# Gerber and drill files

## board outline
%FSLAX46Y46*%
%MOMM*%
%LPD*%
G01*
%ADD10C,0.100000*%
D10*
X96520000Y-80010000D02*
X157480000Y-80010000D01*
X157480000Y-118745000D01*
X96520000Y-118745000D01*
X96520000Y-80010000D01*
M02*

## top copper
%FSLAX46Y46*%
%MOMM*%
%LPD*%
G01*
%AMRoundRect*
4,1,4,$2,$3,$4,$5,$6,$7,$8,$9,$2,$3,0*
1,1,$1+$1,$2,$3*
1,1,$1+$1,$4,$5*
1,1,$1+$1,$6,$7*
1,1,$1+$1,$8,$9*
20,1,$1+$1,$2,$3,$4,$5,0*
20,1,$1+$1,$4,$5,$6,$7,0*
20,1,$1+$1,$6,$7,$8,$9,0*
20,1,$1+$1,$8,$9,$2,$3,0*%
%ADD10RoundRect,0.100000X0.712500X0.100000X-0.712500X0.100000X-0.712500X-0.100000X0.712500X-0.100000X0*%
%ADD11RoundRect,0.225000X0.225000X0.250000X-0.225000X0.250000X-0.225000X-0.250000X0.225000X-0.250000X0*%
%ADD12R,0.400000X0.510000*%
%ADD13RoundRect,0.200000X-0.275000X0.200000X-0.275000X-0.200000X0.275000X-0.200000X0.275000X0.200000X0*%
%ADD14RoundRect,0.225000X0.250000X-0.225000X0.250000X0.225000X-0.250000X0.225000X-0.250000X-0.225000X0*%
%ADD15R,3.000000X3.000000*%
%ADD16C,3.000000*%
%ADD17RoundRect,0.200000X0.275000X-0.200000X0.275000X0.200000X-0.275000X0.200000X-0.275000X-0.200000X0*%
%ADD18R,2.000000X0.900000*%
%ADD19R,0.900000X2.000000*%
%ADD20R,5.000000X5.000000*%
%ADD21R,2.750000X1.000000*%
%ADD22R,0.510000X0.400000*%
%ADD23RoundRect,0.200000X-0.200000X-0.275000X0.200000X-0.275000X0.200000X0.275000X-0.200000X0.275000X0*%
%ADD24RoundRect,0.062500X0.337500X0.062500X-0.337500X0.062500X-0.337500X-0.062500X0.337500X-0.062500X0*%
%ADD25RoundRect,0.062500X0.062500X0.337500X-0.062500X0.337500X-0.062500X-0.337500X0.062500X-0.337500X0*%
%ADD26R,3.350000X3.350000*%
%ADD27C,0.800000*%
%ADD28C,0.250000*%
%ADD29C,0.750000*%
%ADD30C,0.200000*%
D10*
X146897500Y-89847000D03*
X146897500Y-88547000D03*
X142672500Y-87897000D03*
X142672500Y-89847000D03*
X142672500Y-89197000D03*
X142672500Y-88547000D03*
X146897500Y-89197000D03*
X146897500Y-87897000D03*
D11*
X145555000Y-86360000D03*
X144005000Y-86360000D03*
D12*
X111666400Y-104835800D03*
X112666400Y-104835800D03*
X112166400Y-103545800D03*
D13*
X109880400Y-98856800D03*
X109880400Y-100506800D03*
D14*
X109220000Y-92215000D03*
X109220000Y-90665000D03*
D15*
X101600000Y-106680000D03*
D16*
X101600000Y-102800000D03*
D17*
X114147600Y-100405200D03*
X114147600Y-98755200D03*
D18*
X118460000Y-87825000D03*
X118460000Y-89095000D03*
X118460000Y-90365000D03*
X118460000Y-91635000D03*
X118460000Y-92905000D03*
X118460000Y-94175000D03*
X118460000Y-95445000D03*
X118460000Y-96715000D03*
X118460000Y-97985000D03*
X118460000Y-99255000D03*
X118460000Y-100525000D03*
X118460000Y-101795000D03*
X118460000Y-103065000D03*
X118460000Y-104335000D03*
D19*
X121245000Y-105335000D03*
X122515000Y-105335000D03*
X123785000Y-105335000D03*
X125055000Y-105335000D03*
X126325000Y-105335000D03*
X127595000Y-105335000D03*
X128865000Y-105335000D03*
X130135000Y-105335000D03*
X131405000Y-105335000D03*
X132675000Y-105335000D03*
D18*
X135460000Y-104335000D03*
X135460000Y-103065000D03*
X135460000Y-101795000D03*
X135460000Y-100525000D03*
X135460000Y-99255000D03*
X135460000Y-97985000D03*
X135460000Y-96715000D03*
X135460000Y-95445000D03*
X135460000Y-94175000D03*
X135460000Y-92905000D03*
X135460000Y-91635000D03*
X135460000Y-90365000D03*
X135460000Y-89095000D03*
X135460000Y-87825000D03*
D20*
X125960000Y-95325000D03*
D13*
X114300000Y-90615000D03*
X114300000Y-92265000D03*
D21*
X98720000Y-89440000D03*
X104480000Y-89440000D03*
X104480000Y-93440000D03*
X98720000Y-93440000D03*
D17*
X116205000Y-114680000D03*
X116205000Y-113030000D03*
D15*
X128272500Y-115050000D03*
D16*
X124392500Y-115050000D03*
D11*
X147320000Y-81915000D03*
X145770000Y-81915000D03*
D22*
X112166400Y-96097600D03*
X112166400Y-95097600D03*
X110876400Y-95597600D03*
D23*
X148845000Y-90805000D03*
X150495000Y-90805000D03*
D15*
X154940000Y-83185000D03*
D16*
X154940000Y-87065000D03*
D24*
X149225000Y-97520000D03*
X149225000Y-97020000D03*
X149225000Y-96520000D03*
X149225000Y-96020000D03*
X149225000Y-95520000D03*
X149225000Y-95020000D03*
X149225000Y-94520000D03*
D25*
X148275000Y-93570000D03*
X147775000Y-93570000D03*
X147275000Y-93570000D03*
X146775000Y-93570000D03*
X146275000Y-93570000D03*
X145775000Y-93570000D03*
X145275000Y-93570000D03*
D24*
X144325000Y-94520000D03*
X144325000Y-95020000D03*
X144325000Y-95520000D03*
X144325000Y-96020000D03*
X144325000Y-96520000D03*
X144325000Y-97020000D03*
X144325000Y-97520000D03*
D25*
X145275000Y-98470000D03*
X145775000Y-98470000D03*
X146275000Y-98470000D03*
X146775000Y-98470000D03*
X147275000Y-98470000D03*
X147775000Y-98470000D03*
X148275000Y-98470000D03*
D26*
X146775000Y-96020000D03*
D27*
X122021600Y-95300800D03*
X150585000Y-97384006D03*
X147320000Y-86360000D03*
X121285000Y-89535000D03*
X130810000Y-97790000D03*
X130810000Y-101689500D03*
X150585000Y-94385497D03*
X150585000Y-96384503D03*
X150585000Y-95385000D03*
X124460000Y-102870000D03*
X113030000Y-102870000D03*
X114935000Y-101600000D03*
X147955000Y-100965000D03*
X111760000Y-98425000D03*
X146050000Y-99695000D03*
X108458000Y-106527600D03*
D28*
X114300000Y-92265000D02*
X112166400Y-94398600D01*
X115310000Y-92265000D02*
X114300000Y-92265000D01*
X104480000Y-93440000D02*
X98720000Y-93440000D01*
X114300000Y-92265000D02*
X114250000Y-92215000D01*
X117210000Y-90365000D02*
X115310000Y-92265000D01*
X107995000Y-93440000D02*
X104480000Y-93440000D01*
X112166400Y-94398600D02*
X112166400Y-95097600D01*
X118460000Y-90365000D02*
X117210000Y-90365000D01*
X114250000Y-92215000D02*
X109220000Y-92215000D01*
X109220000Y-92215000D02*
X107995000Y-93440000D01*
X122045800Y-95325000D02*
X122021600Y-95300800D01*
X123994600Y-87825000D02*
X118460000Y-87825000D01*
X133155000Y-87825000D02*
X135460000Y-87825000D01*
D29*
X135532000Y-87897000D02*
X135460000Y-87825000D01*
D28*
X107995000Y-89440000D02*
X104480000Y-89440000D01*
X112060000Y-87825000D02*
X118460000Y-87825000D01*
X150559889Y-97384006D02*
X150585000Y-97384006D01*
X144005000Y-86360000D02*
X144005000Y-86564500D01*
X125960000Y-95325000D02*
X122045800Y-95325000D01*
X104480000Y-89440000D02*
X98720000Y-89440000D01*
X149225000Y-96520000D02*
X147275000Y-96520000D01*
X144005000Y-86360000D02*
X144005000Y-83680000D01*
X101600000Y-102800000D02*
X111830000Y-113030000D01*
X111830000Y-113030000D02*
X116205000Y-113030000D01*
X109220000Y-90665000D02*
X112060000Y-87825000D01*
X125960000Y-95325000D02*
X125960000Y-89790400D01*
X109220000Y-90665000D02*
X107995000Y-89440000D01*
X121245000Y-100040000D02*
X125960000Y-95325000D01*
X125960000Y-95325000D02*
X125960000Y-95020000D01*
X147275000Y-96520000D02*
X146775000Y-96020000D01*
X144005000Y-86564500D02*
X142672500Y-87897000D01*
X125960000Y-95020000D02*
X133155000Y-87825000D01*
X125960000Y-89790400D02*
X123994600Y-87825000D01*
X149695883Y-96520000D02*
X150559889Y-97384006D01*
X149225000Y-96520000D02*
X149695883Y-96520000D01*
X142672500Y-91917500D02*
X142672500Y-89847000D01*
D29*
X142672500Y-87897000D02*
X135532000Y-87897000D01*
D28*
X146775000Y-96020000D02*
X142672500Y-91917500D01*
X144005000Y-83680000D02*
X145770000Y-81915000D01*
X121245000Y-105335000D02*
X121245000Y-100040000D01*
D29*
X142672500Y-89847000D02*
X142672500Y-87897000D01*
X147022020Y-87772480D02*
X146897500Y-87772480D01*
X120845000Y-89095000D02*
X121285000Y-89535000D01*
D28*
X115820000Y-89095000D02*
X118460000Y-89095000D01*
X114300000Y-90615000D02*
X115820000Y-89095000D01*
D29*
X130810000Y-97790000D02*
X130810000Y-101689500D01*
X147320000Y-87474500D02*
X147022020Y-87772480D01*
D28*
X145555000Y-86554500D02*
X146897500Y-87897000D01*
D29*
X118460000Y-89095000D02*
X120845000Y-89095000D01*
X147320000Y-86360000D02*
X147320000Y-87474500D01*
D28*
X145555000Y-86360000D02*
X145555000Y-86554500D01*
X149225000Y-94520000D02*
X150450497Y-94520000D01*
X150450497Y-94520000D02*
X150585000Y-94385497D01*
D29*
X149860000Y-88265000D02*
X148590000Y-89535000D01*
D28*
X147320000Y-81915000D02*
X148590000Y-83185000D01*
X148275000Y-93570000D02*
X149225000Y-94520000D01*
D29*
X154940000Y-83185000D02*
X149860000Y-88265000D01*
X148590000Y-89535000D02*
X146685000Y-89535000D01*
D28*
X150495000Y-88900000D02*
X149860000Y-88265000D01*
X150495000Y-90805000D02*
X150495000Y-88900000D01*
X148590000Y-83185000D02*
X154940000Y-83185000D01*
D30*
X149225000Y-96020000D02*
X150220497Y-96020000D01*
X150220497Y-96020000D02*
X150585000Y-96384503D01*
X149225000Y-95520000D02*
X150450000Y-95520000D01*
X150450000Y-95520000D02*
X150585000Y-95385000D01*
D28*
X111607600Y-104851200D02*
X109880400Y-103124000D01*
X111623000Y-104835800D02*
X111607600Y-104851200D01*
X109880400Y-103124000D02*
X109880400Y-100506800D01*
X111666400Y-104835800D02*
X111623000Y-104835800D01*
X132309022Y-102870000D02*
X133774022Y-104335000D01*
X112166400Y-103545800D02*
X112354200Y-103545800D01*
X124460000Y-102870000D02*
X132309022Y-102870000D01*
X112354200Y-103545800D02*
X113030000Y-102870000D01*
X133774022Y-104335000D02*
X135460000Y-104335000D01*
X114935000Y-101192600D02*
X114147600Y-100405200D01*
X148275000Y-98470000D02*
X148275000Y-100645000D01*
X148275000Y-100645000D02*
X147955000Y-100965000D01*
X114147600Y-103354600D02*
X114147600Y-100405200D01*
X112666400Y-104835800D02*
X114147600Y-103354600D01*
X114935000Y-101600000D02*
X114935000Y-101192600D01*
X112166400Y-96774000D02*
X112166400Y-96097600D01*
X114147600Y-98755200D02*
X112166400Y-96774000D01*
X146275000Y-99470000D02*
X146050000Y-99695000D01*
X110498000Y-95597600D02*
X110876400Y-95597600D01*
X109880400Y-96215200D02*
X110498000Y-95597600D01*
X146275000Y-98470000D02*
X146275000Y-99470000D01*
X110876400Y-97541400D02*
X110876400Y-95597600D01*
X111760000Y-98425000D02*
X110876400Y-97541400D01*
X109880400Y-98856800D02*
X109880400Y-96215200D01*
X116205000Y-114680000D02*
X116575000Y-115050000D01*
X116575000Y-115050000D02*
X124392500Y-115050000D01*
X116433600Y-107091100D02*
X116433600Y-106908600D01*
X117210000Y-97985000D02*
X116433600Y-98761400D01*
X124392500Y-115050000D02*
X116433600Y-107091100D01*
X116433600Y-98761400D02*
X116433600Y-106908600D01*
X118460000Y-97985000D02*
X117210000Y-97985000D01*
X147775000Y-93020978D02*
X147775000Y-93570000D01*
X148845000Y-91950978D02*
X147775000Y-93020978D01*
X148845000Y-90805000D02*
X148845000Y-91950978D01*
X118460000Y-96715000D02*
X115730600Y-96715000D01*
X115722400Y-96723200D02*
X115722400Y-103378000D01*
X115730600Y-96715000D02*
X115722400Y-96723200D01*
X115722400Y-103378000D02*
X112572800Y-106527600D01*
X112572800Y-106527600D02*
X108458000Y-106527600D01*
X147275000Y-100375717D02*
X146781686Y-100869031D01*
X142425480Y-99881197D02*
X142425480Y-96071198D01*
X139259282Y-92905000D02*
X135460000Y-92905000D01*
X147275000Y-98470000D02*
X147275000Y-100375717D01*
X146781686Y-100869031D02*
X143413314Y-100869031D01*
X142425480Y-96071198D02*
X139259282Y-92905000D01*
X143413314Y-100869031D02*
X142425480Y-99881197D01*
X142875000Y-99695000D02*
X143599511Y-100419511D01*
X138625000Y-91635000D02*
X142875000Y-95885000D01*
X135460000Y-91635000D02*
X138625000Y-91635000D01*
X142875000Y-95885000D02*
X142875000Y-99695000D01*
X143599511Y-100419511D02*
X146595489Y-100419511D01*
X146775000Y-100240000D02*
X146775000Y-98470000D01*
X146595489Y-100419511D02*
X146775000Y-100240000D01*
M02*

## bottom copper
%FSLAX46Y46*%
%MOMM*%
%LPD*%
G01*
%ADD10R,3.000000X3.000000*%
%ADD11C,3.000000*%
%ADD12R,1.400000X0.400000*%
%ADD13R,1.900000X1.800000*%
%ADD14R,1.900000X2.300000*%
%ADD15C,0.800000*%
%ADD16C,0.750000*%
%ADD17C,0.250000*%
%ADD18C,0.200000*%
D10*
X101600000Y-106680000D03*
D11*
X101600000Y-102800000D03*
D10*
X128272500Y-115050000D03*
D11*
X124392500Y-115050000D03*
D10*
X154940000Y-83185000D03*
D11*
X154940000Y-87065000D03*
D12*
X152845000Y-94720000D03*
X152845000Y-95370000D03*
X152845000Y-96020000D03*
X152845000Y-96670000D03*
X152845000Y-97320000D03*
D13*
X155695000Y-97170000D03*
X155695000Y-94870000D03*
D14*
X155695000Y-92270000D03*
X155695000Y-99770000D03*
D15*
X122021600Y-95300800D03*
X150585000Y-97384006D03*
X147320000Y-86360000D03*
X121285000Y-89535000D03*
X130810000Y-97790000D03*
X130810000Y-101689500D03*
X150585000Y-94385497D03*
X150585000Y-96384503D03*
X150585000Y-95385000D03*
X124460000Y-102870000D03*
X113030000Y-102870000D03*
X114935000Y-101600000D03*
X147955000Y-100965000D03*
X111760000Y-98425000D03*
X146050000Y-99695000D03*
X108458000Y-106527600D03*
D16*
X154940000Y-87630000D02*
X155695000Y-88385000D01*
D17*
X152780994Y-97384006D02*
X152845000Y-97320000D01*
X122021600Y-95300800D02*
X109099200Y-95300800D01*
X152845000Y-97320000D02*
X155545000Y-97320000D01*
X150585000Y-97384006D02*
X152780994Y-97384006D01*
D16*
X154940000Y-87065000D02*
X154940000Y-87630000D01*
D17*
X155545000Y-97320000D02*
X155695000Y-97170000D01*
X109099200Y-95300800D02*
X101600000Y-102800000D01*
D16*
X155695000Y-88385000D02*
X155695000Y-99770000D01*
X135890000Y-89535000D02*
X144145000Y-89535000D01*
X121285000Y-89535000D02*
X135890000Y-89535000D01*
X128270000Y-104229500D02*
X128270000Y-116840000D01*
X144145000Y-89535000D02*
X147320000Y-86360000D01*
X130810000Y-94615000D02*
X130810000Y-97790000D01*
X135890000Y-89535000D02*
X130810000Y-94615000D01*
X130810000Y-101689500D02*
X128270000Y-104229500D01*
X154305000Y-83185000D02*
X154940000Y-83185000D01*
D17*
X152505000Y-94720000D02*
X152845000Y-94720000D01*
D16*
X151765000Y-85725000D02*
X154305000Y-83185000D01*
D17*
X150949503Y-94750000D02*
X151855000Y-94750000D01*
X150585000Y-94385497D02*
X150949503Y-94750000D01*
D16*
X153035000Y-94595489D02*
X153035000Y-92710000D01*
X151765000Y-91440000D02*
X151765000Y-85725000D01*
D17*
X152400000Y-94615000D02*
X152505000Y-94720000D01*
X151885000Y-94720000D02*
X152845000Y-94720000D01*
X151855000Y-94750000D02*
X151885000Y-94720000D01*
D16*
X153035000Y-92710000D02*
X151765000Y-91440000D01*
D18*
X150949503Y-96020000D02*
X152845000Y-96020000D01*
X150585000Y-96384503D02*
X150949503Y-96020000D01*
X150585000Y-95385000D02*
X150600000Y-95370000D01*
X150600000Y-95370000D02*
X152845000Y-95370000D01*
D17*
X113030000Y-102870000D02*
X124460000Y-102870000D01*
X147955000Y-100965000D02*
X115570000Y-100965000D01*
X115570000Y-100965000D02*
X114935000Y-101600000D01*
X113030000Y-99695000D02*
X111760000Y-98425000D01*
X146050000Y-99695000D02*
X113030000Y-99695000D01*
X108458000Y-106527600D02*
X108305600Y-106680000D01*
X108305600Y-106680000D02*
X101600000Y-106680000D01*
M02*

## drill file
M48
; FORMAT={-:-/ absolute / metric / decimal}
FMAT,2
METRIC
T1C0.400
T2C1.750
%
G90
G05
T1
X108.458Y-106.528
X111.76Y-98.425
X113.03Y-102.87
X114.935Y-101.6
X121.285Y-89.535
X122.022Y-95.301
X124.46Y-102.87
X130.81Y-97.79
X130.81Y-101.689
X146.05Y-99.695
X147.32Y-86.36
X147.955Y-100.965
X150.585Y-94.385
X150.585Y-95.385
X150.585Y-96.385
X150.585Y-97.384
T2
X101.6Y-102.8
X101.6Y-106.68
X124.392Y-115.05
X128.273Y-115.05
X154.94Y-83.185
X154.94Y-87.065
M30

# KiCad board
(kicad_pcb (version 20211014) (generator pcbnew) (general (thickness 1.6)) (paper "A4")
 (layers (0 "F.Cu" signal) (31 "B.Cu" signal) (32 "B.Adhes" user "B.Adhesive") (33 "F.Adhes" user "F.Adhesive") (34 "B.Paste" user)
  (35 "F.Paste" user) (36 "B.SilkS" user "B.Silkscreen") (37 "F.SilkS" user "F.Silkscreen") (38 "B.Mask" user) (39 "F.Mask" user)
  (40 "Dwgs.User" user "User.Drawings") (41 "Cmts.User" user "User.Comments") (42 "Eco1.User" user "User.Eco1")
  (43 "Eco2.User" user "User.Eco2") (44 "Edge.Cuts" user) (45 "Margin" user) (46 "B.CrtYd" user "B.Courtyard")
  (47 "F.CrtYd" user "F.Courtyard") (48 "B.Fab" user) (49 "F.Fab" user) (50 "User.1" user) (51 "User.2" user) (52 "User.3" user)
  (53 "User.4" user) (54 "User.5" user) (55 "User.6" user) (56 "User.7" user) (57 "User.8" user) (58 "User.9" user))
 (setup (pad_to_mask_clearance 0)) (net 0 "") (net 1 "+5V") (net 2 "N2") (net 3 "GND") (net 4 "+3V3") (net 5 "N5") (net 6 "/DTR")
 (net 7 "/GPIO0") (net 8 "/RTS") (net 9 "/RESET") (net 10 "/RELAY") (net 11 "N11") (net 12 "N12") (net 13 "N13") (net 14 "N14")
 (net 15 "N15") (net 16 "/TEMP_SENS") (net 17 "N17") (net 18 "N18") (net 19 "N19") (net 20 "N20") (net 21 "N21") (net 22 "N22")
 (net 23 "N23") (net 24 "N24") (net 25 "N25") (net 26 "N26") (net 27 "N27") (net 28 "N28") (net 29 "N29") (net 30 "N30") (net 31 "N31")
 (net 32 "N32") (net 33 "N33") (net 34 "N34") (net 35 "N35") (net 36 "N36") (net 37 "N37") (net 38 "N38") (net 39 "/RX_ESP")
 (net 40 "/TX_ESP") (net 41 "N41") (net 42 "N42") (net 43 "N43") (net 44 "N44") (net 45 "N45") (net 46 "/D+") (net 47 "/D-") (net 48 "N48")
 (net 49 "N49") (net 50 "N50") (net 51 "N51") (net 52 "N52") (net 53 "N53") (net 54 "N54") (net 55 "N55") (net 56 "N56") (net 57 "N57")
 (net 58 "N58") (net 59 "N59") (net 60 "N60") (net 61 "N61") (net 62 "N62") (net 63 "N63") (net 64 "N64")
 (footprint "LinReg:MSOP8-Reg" (layer "F.Cu") (at 144.78 88.9 180)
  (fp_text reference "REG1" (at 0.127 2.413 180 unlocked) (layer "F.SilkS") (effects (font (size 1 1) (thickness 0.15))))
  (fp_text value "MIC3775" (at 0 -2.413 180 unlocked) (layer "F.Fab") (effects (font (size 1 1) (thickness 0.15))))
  (pad "EN" smd roundrect (at -2.1175 -0.947 180) (size 1.625 0.4) (layers "F.Cu" "F.Paste" "F.Mask") (roundrect_rratio 0.25) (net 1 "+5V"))
  (pad "FLG" smd roundrect (at -2.1175 0.353 180) (size 1.625 0.4) (layers "F.Cu" "F.Paste" "F.Mask") (roundrect_rratio 0.25) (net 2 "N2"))
  (pad "GND" smd roundrect (at 2.1075 1.003 180) (size 1.625 0.4) (layers "F.Cu" "F.Paste" "F.Mask") (roundrect_rratio 0.25) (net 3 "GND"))
  (pad "GND" smd roundrect (at 2.1075 -0.947 180) (size 1.625 0.4) (layers "F.Cu" "F.Paste" "F.Mask") (roundrect_rratio 0.25) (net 3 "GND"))
  (pad "GND" smd roundrect (at 2.1075 -0.297 180) (size 1.625 0.4) (layers "F.Cu" "F.Paste" "F.Mask") (roundrect_rratio 0.25) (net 3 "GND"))
  (pad "GND" smd roundrect (at 2.1075 0.353 180) (size 1.625 0.4) (layers "F.Cu" "F.Paste" "F.Mask") (roundrect_rratio 0.25) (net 3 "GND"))
  (pad "IN" smd roundrect (at -2.1175 -0.297 180) (size 1.625 0.4) (layers "F.Cu" "F.Paste" "F.Mask") (roundrect_rratio 0.25) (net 1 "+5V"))
  (pad "OUT" smd roundrect (at -2.1175 1.003 180) (size 1.625 0.4) (layers "F.Cu" "F.Paste" "F.Mask") (roundrect_rratio 0.25) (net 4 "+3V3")))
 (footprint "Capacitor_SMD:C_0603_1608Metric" (layer "F.Cu") (at 144.78 86.36 180)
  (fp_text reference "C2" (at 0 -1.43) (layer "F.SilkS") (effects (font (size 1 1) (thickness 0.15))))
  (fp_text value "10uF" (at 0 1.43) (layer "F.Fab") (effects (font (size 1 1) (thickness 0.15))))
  (pad "1" smd roundrect locked (at -0.775 0 180) (size 0.9 0.95) (layers "F.Cu" "F.Paste" "F.Mask") (roundrect_rratio 0.25) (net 4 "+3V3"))
  (pad "2" smd roundrect locked (at 0.775 0 180) (size 0.9 0.95) (layers "F.Cu" "F.Paste" "F.Mask") (roundrect_rratio 0.25) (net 3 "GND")))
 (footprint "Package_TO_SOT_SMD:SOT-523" (layer "F.Cu") (at 112.1664 104.1908 90)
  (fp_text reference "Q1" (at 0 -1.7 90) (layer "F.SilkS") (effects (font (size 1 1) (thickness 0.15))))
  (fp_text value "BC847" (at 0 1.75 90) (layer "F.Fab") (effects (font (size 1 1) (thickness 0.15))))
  (pad "1" smd rect locked (at -0.645 -0.5 270) (size 0.51 0.4) (layers "F.Cu" "F.Paste" "F.Mask") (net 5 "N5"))
  (pad "2" smd rect locked (at -0.645 0.5 270) (size 0.51 0.4) (layers "F.Cu" "F.Paste" "F.Mask") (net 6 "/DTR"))
  (pad "3" smd rect locked (at 0.645 0 270) (size 0.51 0.4) (layers "F.Cu" "F.Paste" "F.Mask") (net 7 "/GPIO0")))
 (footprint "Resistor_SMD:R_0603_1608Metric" (layer "F.Cu") (at 109.8804 99.6818 -90)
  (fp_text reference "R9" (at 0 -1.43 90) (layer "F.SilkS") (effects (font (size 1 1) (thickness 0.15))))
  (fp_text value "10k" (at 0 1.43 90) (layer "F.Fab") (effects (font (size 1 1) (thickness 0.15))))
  (pad "1" smd roundrect locked (at -0.825 0 270) (size 0.8 0.95) (layers "F.Cu" "F.Paste" "F.Mask") (roundrect_rratio 0.25) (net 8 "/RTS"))
  (pad "2" smd roundrect locked (at 0.825 0 270) (size 0.8 0.95) (layers "F.Cu" "F.Paste" "F.Mask") (roundrect_rratio 0.25) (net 5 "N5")))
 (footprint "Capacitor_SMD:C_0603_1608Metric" (layer "F.Cu") (at 109.22 91.44 90)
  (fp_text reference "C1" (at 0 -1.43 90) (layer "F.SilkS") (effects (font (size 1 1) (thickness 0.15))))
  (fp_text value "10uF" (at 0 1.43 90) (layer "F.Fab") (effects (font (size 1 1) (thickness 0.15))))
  (pad "1" smd roundrect locked (at -0.775 0 90) (size 0.9 0.95) (layers "F.Cu" "F.Paste" "F.Mask") (roundrect_rratio 0.25) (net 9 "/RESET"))
  (pad "2" smd roundrect locked (at 0.775 0 90) (size 0.9 0.95) (layers "F.Cu" "F.Paste" "F.Mask") (roundrect_rratio 0.25) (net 3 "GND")))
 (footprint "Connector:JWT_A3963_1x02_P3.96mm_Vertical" (layer "F.Cu") (at 101.6 106.68 90)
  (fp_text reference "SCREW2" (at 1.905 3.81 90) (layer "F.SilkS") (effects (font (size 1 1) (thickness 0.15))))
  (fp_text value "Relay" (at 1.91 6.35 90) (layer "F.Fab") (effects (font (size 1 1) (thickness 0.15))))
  (pad "1" thru_hole rect locked (at 0 0 90) (size 3 3) (drill 1.75) (layers *.Cu *.Mask) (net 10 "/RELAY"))
  (pad "2" thru_hole circle locked (at 3.88 0 90) (size 3 3) (drill 1.75) (layers *.Cu *.Mask) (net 3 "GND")))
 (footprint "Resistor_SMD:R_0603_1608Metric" (layer "F.Cu") (at 114.1476 99.5802 90)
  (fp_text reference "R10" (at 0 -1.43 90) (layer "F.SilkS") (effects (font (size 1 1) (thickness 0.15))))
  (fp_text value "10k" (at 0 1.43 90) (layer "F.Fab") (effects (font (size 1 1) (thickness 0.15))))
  (pad "1" smd roundrect locked (at -0.825 0 90) (size 0.8 0.95) (layers "F.Cu" "F.Paste" "F.Mask") (roundrect_rratio 0.25) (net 6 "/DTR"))
  (pad "2" smd roundrect locked (at 0.825 0 90) (size 0.8 0.95) (layers "F.Cu" "F.Paste" "F.Mask") (roundrect_rratio 0.25) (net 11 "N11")))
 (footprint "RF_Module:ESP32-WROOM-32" (layer "F.Cu") (at 126.96 96.08)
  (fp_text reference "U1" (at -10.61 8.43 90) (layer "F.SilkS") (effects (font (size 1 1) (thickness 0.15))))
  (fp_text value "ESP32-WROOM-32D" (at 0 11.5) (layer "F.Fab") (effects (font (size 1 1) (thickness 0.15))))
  (pad "1" smd rect locked (at -8.5 -8.255) (size 2 0.9) (layers "F.Cu" "F.Paste" "F.Mask") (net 3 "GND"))
  (pad "2" smd rect locked (at -8.5 -6.985) (size 2 0.9) (layers "F.Cu" "F.Paste" "F.Mask") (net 4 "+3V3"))
  (pad "3" smd rect locked (at -8.5 -5.715) (size 2 0.9) (layers "F.Cu" "F.Paste" "F.Mask") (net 9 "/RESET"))
  (pad "4" smd rect locked (at -8.5 -4.445) (size 2 0.9) (layers "F.Cu" "F.Paste" "F.Mask") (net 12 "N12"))
  (pad "5" smd rect locked (at -8.5 -3.175) (size 2 0.9) (layers "F.Cu" "F.Paste" "F.Mask") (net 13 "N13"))
  (pad "6" smd rect locked (at -8.5 -1.905) (size 2 0.9) (layers "F.Cu" "F.Paste" "F.Mask") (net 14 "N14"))
  (pad "7" smd rect locked (at -8.5 -0.635) (size 2 0.9) (layers "F.Cu" "F.Paste" "F.Mask") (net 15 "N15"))
  (pad "8" smd rect locked (at -8.5 0.635) (size 2 0.9) (layers "F.Cu" "F.Paste" "F.Mask") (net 10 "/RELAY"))
  (pad "9" smd rect locked (at -8.5 1.905) (size 2 0.9) (layers "F.Cu" "F.Paste" "F.Mask") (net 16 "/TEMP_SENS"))
  (pad "10" smd rect locked (at -8.5 3.175) (size 2 0.9) (layers "F.Cu" "F.Paste" "F.Mask") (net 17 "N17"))
  (pad "11" smd rect locked (at -8.5 4.445) (size 2 0.9) (layers "F.Cu" "F.Paste" "F.Mask") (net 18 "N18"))
  (pad "12" smd rect locked (at -8.5 5.715) (size 2 0.9) (layers "F.Cu" "F.Paste" "F.Mask") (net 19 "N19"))
  (pad "13" smd rect locked (at -8.5 6.985) (size 2 0.9) (layers "F.Cu" "F.Paste" "F.Mask") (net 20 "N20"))
  (pad "14" smd rect locked (at -8.5 8.255) (size 2 0.9) (layers "F.Cu" "F.Paste" "F.Mask") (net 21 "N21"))
  (pad "15" smd rect locked (at -5.715 9.255 90) (size 2 0.9) (layers "F.Cu" "F.Paste" "F.Mask") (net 3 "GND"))
  (pad "16" smd rect locked (at -4.445 9.255 90) (size 2 0.9) (layers "F.Cu" "F.Paste" "F.Mask") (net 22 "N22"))
  (pad "17" smd rect locked (at -3.175 9.255 90) (size 2 0.9) (layers "F.Cu" "F.Paste" "F.Mask") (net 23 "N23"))
  (pad "18" smd rect locked (at -1.905 9.255 90) (size 2 0.9) (layers "F.Cu" "F.Paste" "F.Mask") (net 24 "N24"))
  (pad "19" smd rect locked (at -0.635 9.255 90) (size 2 0.9) (layers "F.Cu" "F.Paste" "F.Mask") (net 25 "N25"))
  (pad "20" smd rect locked (at 0.635 9.255 90) (size 2 0.9) (layers "F.Cu" "F.Paste" "F.Mask") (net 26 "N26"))
  (pad "21" smd rect locked (at 1.905 9.255 90) (size 2 0.9) (layers "F.Cu" "F.Paste" "F.Mask") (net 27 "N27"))
  (pad "22" smd rect locked (at 3.175 9.255 90) (size 2 0.9) (layers "F.Cu" "F.Paste" "F.Mask") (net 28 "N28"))
  (pad "23" smd rect locked (at 4.445 9.255 90) (size 2 0.9) (layers "F.Cu" "F.Paste" "F.Mask") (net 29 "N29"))
  (pad "24" smd rect locked (at 5.715 9.255 90) (size 2 0.9) (layers "F.Cu" "F.Paste" "F.Mask") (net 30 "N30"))
  (pad "25" smd rect locked (at 8.5 8.255) (size 2 0.9) (layers "F.Cu" "F.Paste" "F.Mask") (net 7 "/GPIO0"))
  (pad "26" smd rect locked (at 8.5 6.985) (size 2 0.9) (layers "F.Cu" "F.Paste" "F.Mask") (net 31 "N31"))
  (pad "27" smd rect locked (at 8.5 5.715) (size 2 0.9) (layers "F.Cu" "F.Paste" "F.Mask") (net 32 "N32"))
  (pad "28" smd rect locked (at 8.5 4.445) (size 2 0.9) (layers "F.Cu" "F.Paste" "F.Mask") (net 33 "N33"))
  (pad "29" smd rect locked (at 8.5 3.175) (size 2 0.9) (layers "F.Cu" "F.Paste" "F.Mask") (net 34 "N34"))
  (pad "30" smd rect locked (at 8.5 1.905) (size 2 0.9) (layers "F.Cu" "F.Paste" "F.Mask") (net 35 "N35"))
  (pad "31" smd rect locked (at 8.5 0.635) (size 2 0.9) (layers "F.Cu" "F.Paste" "F.Mask") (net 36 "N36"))
  (pad "32" smd rect locked (at 8.5 -0.635) (size 2 0.9) (layers "F.Cu" "F.Paste" "F.Mask") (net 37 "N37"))
  (pad "33" smd rect locked (at 8.5 -1.905) (size 2 0.9) (layers "F.Cu" "F.Paste" "F.Mask") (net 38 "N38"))
  (pad "34" smd rect locked (at 8.5 -3.175) (size 2 0.9) (layers "F.Cu" "F.Paste" "F.Mask") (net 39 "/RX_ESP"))
  (pad "35" smd rect locked (at 8.5 -4.445) (size 2 0.9) (layers "F.Cu" "F.Paste" "F.Mask") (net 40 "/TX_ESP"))
  (pad "36" smd rect locked (at 8.5 -5.715) (size 2 0.9) (layers "F.Cu" "F.Paste" "F.Mask") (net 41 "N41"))
  (pad "37" smd rect locked (at 8.5 -6.985) (size 2 0.9) (layers "F.Cu" "F.Paste" "F.Mask") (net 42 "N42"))
  (pad "38" smd rect locked (at 8.5 -8.255) (size 2 0.9) (layers "F.Cu" "F.Paste" "F.Mask") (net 3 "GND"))
  (pad "39" smd rect locked (at -1 -0.755) (size 5 5) (layers "F.Cu" "F.Paste" "F.Mask") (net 3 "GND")))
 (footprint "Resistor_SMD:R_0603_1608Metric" (layer "F.Cu") (at 114.3 91.44 -90)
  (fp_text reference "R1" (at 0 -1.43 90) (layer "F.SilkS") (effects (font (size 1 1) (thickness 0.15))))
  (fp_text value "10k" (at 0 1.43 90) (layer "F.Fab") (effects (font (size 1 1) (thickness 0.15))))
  (pad "1" smd roundrect locked (at -0.825 0 270) (size 0.8 0.95) (layers "F.Cu" "F.Paste" "F.Mask") (roundrect_rratio 0.25) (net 4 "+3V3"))
  (pad "2" smd roundrect locked (at 0.825 0 270) (size 0.8 0.95) (layers "F.Cu" "F.Paste" "F.Mask") (roundrect_rratio 0.25) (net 9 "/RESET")))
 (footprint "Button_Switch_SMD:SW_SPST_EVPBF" (layer "F.Cu") (at 101.6 91.44)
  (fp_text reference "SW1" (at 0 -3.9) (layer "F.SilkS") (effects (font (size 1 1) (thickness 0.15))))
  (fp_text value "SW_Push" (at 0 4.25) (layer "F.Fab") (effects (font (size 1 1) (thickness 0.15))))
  (pad "1" smd rect locked (at -2.88 -2) (size 2.75 1) (layers "F.Cu" "F.Paste" "F.Mask") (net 3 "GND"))
  (pad "1" smd rect locked (at 2.88 -2) (size 2.75 1) (layers "F.Cu" "F.Paste" "F.Mask") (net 3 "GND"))
  (pad "2" smd rect locked (at 2.88 2) (size 2.75 1) (layers "F.Cu" "F.Paste" "F.Mask") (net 9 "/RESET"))
  (pad "2" smd rect locked (at -2.88 2) (size 2.75 1) (layers "F.Cu" "F.Paste" "F.Mask") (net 9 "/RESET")))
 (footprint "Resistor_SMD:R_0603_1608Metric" (layer "F.Cu") (at 116.205 113.855 90)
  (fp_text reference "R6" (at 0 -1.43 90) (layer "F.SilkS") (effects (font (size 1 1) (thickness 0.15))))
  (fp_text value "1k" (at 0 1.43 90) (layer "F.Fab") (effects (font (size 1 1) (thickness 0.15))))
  (pad "1" smd roundrect locked (at -0.825 0 90) (size 0.8 0.95) (layers "F.Cu" "F.Paste" "F.Mask") (roundrect_rratio 0.25)
   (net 16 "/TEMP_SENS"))
  (pad "2" smd roundrect locked (at 0.825 0 90) (size 0.8 0.95) (layers "F.Cu" "F.Paste" "F.Mask") (roundrect_rratio 0.25) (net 3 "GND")))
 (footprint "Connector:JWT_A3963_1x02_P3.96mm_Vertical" (layer "F.Cu") (at 128.2725 115.05 180)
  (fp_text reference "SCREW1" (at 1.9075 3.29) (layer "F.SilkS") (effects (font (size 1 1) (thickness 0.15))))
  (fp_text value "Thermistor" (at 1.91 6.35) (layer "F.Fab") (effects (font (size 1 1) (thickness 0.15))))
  (pad "1" thru_hole rect locked (at 0 0 180) (size 3 3) (drill 1.75) (layers *.Cu *.Mask) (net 4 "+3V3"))
  (pad "2" thru_hole circle locked (at 3.88 0 180) (size 3 3) (drill 1.75) (layers *.Cu *.Mask) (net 16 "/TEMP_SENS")))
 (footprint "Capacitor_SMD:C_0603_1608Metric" (layer "F.Cu") (at 146.545 81.915 180)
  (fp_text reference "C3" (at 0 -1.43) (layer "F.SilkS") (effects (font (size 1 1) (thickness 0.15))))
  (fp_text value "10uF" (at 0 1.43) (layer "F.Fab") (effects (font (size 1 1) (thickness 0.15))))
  (pad "1" smd roundrect locked (at -0.775 0 180) (size 0.9 0.95) (layers "F.Cu" "F.Paste" "F.Mask") (roundrect_rratio 0.25) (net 1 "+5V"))
  (pad "2" smd roundrect locked (at 0.775 0 180) (size 0.9 0.95) (layers "F.Cu" "F.Paste" "F.Mask") (roundrect_rratio 0.25) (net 3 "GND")))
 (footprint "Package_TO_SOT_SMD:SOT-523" (layer "F.Cu") (at 111.5214 95.5976 180)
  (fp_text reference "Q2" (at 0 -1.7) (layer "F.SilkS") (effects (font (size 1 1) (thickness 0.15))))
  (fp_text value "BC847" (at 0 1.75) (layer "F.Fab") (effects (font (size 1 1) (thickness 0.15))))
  (pad "1" smd rect locked (at -0.645 -0.5) (size 0.51 0.4) (layers "F.Cu" "F.Paste" "F.Mask") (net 11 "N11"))
  (pad "2" smd rect locked (at -0.645 0.5) (size 0.51 0.4) (layers "F.Cu" "F.Paste" "F.Mask") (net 9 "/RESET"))
  (pad "3" smd rect locked (at 0.645 0) (size 0.51 0.4) (layers "F.Cu" "F.Paste" "F.Mask") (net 8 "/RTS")))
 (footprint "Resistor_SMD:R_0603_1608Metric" (layer "F.Cu") (at 149.67 90.805)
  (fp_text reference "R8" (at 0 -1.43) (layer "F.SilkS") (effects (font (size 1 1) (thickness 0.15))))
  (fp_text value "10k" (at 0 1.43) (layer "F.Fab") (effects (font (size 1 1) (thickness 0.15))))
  (pad "1" smd roundrect locked (at -0.825 0) (size 0.8 0.95) (layers "F.Cu" "F.Paste" "F.Mask") (roundrect_rratio 0.25) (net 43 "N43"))
  (pad "2" smd roundrect locked (at 0.825 0) (size 0.8 0.95) (layers "F.Cu" "F.Paste" "F.Mask") (roundrect_rratio 0.25) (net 1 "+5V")))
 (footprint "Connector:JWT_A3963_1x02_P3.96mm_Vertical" (layer "F.Cu") (at 154.94 83.185 -90)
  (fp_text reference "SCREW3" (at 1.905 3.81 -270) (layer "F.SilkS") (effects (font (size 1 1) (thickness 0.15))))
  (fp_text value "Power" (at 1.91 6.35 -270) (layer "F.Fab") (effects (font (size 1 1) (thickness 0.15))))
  (pad "1" thru_hole rect locked (at 0 0 270) (size 3 3) (drill 1.75) (layers *.Cu *.Mask) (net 1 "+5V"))
  (pad "2" thru_hole circle locked (at 3.88 0 270) (size 3 3) (drill 1.75) (layers *.Cu *.Mask) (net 3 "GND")))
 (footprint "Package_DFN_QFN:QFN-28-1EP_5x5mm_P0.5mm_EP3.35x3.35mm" (layer "F.Cu") (at 146.775 96.02 180)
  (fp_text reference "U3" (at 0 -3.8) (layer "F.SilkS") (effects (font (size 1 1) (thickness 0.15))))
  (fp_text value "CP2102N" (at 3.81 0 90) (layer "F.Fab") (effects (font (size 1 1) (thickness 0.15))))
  (pad "" smd roundrect locked (at 1.12 1.12 180) (size 0.9 0.9) (layers "F.Paste") (roundrect_rratio 0.25))
  (pad "" smd roundrect locked (at -1.12 -1.12 180) (size 0.9 0.9) (layers "F.Paste") (roundrect_rratio 0.25))
  (pad "" smd roundrect locked (at 0 -1.12 180) (size 0.9 0.9) (layers "F.Paste") (roundrect_rratio 0.25))
  (pad "" smd roundrect locked (at 1.12 0 180) (size 0.9 0.9) (layers "F.Paste") (roundrect_rratio 0.25))
  (pad "" smd roundrect locked (at 0 1.12 180) (size 0.9 0.9) (layers "F.Paste") (roundrect_rratio 0.25))
  (pad "" smd roundrect locked (at 0 0 180) (size 0.9 0.9) (layers "F.Paste") (roundrect_rratio 0.25))
  (pad "" smd roundrect locked (at -1.12 1.12 180) (size 0.9 0.9) (layers "F.Paste") (roundrect_rratio 0.25))
  (pad "" smd roundrect locked (at 1.12 -1.12 180) (size 0.9 0.9) (layers "F.Paste") (roundrect_rratio 0.25))
  (pad "" smd roundrect locked (at -1.12 0 180) (size 0.9 0.9) (layers "F.Paste") (roundrect_rratio 0.25))
  (pad "1" smd roundrect locked (at -2.45 -1.5 180) (size 0.8 0.25) (layers "F.Cu" "F.Paste" "F.Mask") (roundrect_rratio 0.25)
   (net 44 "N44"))
  (pad "2" smd roundrect locked (at -2.45 -1 180) (size 0.8 0.25) (layers "F.Cu" "F.Paste" "F.Mask") (roundrect_rratio 0.25) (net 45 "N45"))
  (pad "3" smd roundrect locked (at -2.45 -0.5 180) (size 0.8 0.25) (layers "F.Cu" "F.Paste" "F.Mask") (roundrect_rratio 0.25) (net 3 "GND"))
  (pad "4" smd roundrect locked (at -2.45 0 180) (size 0.8 0.25) (layers "F.Cu" "F.Paste" "F.Mask") (roundrect_rratio 0.25) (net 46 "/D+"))
  (pad "5" smd roundrect locked (at -2.45 0.5 180) (size 0.8 0.25) (layers "F.Cu" "F.Paste" "F.Mask") (roundrect_rratio 0.25) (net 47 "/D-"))
  (pad "6" smd roundrect locked (at -2.45 1 180) (size 0.8 0.25) (layers "F.Cu" "F.Paste" "F.Mask") (roundrect_rratio 0.25) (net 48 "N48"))
  (pad "7" smd roundrect locked (at -2.45 1.5 180) (size 0.8 0.25) (layers "F.Cu" "F.Paste" "F.Mask") (roundrect_rratio 0.25) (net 1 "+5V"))
  (pad "8" smd roundrect locked (at -1.5 2.45 180) (size 0.25 0.8) (layers "F.Cu" "F.Paste" "F.Mask") (roundrect_rratio 0.25) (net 1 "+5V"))
  (pad "9" smd roundrect locked (at -1 2.45 180) (size 0.25 0.8) (layers "F.Cu" "F.Paste" "F.Mask") (roundrect_rratio 0.25) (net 43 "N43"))
  (pad "10" smd roundrect locked (at -0.5 2.45 180) (size 0.25 0.8) (layers "F.Cu" "F.Paste" "F.Mask") (roundrect_rratio 0.25)
   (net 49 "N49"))
  (pad "11" smd roundrect locked (at 0 2.45 180) (size 0.25 0.8) (layers "F.Cu" "F.Paste" "F.Mask") (roundrect_rratio 0.25) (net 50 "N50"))
  (pad "12" smd roundrect locked (at 0.5 2.45 180) (size 0.25 0.8) (layers "F.Cu" "F.Paste" "F.Mask") (roundrect_rratio 0.25) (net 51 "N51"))
  (pad "13" smd roundrect locked (at 1 2.45 180) (size 0.25 0.8) (layers "F.Cu" "F.Paste" "F.Mask") (roundrect_rratio 0.25) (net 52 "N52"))
  (pad "14" smd roundrect locked (at 1.5 2.45 180) (size 0.25 0.8) (layers "F.Cu" "F.Paste" "F.Mask") (roundrect_rratio 0.25) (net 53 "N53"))
  (pad "15" smd roundrect locked (at 2.45 1.5 180) (size 0.8 0.25) (layers "F.Cu" "F.Paste" "F.Mask") (roundrect_rratio 0.25) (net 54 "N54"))
  (pad "16" smd roundrect locked (at 2.45 1 180) (size 0.8 0.25) (layers "F.Cu" "F.Paste" "F.Mask") (roundrect_rratio 0.25) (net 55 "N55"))
  (pad "17" smd roundrect locked (at 2.45 0.5 180) (size 0.8 0.25) (layers "F.Cu" "F.Paste" "F.Mask") (roundrect_rratio 0.25) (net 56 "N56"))
  (pad "18" smd roundrect locked (at 2.45 0 180) (size 0.8 0.25) (layers "F.Cu" "F.Paste" "F.Mask") (roundrect_rratio 0.25) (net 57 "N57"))
  (pad "19" smd roundrect locked (at 2.45 -0.5 180) (size 0.8 0.25) (layers "F.Cu" "F.Paste" "F.Mask") (roundrect_rratio 0.25)
   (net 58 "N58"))
  (pad "20" smd roundrect locked (at 2.45 -1 180) (size 0.8 0.25) (layers "F.Cu" "F.Paste" "F.Mask") (roundrect_rratio 0.25) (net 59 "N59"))
  (pad "21" smd roundrect locked (at 2.45 -1.5 180) (size 0.8 0.25) (layers "F.Cu" "F.Paste" "F.Mask") (roundrect_rratio 0.25)
   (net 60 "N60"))
  (pad "22" smd roundrect locked (at 1.5 -2.45 180) (size 0.25 0.8) (layers "F.Cu" "F.Paste" "F.Mask") (roundrect_rratio 0.25)
   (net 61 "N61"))
  (pad "23" smd roundrect locked (at 1 -2.45 180) (size 0.25 0.8) (layers "F.Cu" "F.Paste" "F.Mask") (roundrect_rratio 0.25) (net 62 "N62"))
  (pad "24" smd roundrect locked (at 0.5 -2.45 180) (size 0.25 0.8) (layers "F.Cu" "F.Paste" "F.Mask") (roundrect_rratio 0.25)
   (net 8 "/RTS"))
  (pad "25" smd roundrect locked (at 0 -2.45 180) (size 0.25 0.8) (layers "F.Cu" "F.Paste" "F.Mask") (roundrect_rratio 0.25)
   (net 40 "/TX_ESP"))
  (pad "26" smd roundrect locked (at -0.5 -2.45 180) (size 0.25 0.8) (layers "F.Cu" "F.Paste" "F.Mask") (roundrect_rratio 0.25)
   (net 39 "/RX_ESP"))
  (pad "27" smd roundrect locked (at -1 -2.45 180) (size 0.25 0.8) (layers "F.Cu" "F.Paste" "F.Mask") (roundrect_rratio 0.25) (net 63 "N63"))
  (pad "28" smd roundrect locked (at -1.5 -2.45 180) (size 0.25 0.8) (layers "F.Cu" "F.Paste" "F.Mask") (roundrect_rratio 0.25)
   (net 6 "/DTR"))
  (pad "29" smd rect locked (at 0 0 180) (size 3.35 3.35) (layers "F.Cu" "F.Mask") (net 3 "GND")))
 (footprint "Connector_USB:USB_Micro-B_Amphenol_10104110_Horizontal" (layer "B.Cu") (at 154.395 96.02 -90)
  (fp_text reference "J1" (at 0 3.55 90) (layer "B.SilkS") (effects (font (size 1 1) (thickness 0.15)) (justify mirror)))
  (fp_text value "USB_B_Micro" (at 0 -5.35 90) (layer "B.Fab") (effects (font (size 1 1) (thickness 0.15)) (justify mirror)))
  (pad "1" smd rect locked (at -1.3 1.55 270) (size 0.4 1.4) (layers "B.Cu" "B.Paste" "B.Mask") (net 1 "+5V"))
  (pad "2" smd rect locked (at -0.65 1.55 270) (size 0.4 1.4) (layers "B.Cu" "B.Paste" "B.Mask") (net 47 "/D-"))
  (pad "3" smd rect locked (at 0 1.55 270) (size 0.4 1.4) (layers "B.Cu" "B.Paste" "B.Mask") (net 46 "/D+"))
  (pad "4" smd rect locked (at 0.65 1.55 270) (size 0.4 1.4) (layers "B.Cu" "B.Paste" "B.Mask") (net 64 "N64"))
  (pad "5" smd rect locked (at 1.3 1.55 270) (size 0.4 1.4) (layers "B.Cu" "B.Paste" "B.Mask") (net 3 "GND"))
  (pad "6" smd rect locked (at 1.15 -1.3 270) (size 1.8 1.9) (layers "B.Cu" "B.Paste" "B.Mask") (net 3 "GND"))
  (pad "6" smd rect locked (at -1.15 -1.3 270) (size 1.8 1.9) (layers "B.Cu" "B.Paste" "B.Mask") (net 3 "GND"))
  (pad "6" smd rect locked (at -3.75 -1.3 270) (size 2.3 1.9) (layers "B.Cu" "B.Paste" "B.Mask") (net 3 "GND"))
  (pad "6" smd rect locked (at 3.75 -1.3 270) (size 2.3 1.9) (layers "B.Cu" "B.Paste" "B.Mask") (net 3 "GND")))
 (gr_rect (start 96.52 80.01) (end 157.48 118.745) (layer "Edge.Cuts") (width 0.1) (fill none))
 (segment (start 114.3 92.265) (end 112.1664 94.3986) (width 0.25) (layer "F.Cu") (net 9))
 (segment (start 115.31 92.265) (end 114.3 92.265) (width 0.25) (layer "F.Cu") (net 9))
 (segment (start 104.48 93.44) (end 98.72 93.44) (width 0.25) (layer "F.Cu") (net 9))
 (segment (start 114.3 92.265) (end 114.25 92.215) (width 0.25) (layer "F.Cu") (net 9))
 (segment (start 117.21 90.365) (end 115.31 92.265) (width 0.25) (layer "F.Cu") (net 9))
 (segment (start 107.995 93.44) (end 104.48 93.44) (width 0.25) (layer "F.Cu") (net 9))
 (segment (start 112.1664 94.3986) (end 112.1664 95.0976) (width 0.25) (layer "F.Cu") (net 9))
 (segment (start 118.46 90.365) (end 117.21 90.365) (width 0.25) (layer "F.Cu") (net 9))
 (segment (start 114.25 92.215) (end 109.22 92.215) (width 0.25) (layer "F.Cu") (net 9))
 (segment (start 109.22 92.215) (end 107.995 93.44) (width 0.25) (layer "F.Cu") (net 9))
 (segment (start 122.0458 95.325) (end 122.0216 95.3008) (width 0.25) (layer "F.Cu") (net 3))
 (segment (start 123.9946 87.825) (end 118.46 87.825) (width 0.25) (layer "F.Cu") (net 3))
 (segment (start 133.155 87.825) (end 135.46 87.825) (width 0.25) (layer "F.Cu") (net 3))
 (segment (start 135.532 87.897) (end 135.46 87.825) (width 0.75) (layer "F.Cu") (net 3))
 (segment (start 107.995 89.44) (end 104.48 89.44) (width 0.25) (layer "F.Cu") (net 3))
 (segment (start 112.06 87.825) (end 118.46 87.825) (width 0.25) (layer "F.Cu") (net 3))
 (segment (start 150.559889 97.384006) (end 150.585 97.384006) (width 0.25) (layer "F.Cu") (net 3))
 (segment (start 144.005 86.36) (end 144.005 86.5645) (width 0.25) (layer "F.Cu") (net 3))
 (segment (start 125.96 95.325) (end 122.0458 95.325) (width 0.25) (layer "F.Cu") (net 3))
 (segment (start 104.48 89.44) (end 98.72 89.44) (width 0.25) (layer "F.Cu") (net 3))
 (segment (start 149.225 96.52) (end 147.275 96.52) (width 0.25) (layer "F.Cu") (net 3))
 (segment (start 144.005 86.36) (end 144.005 83.68) (width 0.25) (layer "F.Cu") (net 3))
 (segment (start 101.6 102.8) (end 111.83 113.03) (width 0.25) (layer "F.Cu") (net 3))
 (segment (start 111.83 113.03) (end 116.205 113.03) (width 0.25) (layer "F.Cu") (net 3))
 (segment (start 109.22 90.665) (end 112.06 87.825) (width 0.25) (layer "F.Cu") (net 3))
 (segment (start 125.96 95.325) (end 125.96 89.7904) (width 0.25) (layer "F.Cu") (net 3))
 (segment (start 109.22 90.665) (end 107.995 89.44) (width 0.25) (layer "F.Cu") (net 3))
 (segment (start 121.245 100.04) (end 125.96 95.325) (width 0.25) (layer "F.Cu") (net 3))
 (segment (start 125.96 95.325) (end 125.96 95.02) (width 0.25) (layer "F.Cu") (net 3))
 (segment (start 147.275 96.52) (end 146.775 96.02) (width 0.25) (layer "F.Cu") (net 3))
 (segment (start 144.005 86.5645) (end 142.6725 87.897) (width 0.25) (layer "F.Cu") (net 3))
 (segment (start 125.96 95.02) (end 133.155 87.825) (width 0.25) (layer "F.Cu") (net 3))
 (segment (start 125.96 89.7904) (end 123.9946 87.825) (width 0.25) (layer "F.Cu") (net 3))
 (segment (start 149.695883 96.52) (end 150.559889 97.384006) (width 0.25) (layer "F.Cu") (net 3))
 (segment (start 149.225 96.52) (end 149.695883 96.52) (width 0.25) (layer "F.Cu") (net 3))
 (segment (start 142.6725 91.9175) (end 142.6725 89.847) (width 0.25) (layer "F.Cu") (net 3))
 (segment (start 142.6725 87.897) (end 135.532 87.897) (width 0.75) (layer "F.Cu") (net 3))
 (segment (start 146.775 96.02) (end 142.6725 91.9175) (width 0.25) (layer "F.Cu") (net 3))
 (segment (start 144.005 83.68) (end 145.77 81.915) (width 0.25) (layer "F.Cu") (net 3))
 (segment (start 121.245 105.335) (end 121.245 100.04) (width 0.25) (layer "F.Cu") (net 3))
 (segment (start 142.6725 89.847) (end 142.6725 87.897) (width 0.75) (layer "F.Cu") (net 3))
 (via (at 122.0216 95.3008) (size 0.8) (drill 0.4) (layers "F.Cu" "B.Cu") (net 3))
 (via (at 150.585 97.384006) (size 0.8) (drill 0.4) (layers "F.Cu" "B.Cu") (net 3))
 (segment (start 154.94 87.63) (end 155.695 88.385) (width 0.75) (layer "B.Cu") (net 3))
 (segment (start 152.780994 97.384006) (end 152.845 97.32) (width 0.25) (layer "B.Cu") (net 3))
 (segment (start 122.0216 95.3008) (end 109.0992 95.3008) (width 0.25) (layer "B.Cu") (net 3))
 (segment (start 152.845 97.32) (end 155.545 97.32) (width 0.25) (layer "B.Cu") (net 3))
 (segment (start 150.585 97.384006) (end 152.780994 97.384006) (width 0.25) (layer "B.Cu") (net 3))
 (segment (start 154.94 87.065) (end 154.94 87.63) (width 0.75) (layer "B.Cu") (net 3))
 (segment (start 155.545 97.32) (end 155.695 97.17) (width 0.25) (layer "B.Cu") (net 3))
 (segment (start 109.0992 95.3008) (end 101.6 102.8) (width 0.25) (layer "B.Cu") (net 3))
 (segment (start 155.695 88.385) (end 155.695 99.77) (width 0.75) (layer "B.Cu") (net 3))
 (segment (start 147.02202 87.77248) (end 146.8975 87.77248) (width 0.75) (layer "F.Cu") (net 4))
 (segment (start 120.845 89.095) (end 121.285 89.535) (width 0.75) (layer "F.Cu") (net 4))
 (segment (start 115.82 89.095) (end 118.46 89.095) (width 0.25) (layer "F.Cu") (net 4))
 (segment (start 114.3 90.615) (end 115.82 89.095) (width 0.25) (layer "F.Cu") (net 4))
 (segment (start 130.81 97.79) (end 130.81 101.6895) (width 0.75) (layer "F.Cu") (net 4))
 (segment (start 147.32 87.4745) (end 147.02202 87.77248) (width 0.75) (layer "F.Cu") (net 4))
 (segment (start 145.555 86.5545) (end 146.8975 87.897) (width 0.25) (layer "F.Cu") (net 4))
 (segment (start 118.46 89.095) (end 120.845 89.095) (width 0.75) (layer "F.Cu") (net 4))
 (segment (start 147.32 86.36) (end 147.32 87.4745) (width 0.75) (layer "F.Cu") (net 4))
 (segment (start 145.555 86.36) (end 145.555 86.5545) (width 0.25) (layer "F.Cu") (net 4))
 (via (at 147.32 86.36) (size 0.8) (drill 0.4) (layers "F.Cu" "B.Cu") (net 4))
 (via (at 121.285 89.535) (size 0.8) (drill 0.4) (layers "F.Cu" "B.Cu") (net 4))
 (via (at 130.81 97.79) (size 0.8) (drill 0.4) (layers "F.Cu" "B.Cu") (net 4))
 (via (at 130.81 101.6895) (size 0.8) (drill 0.4) (layers "F.Cu" "B.Cu") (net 4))
 (segment (start 135.89 89.535) (end 144.145 89.535) (width 0.75) (layer "B.Cu") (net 4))
 (segment (start 121.285 89.535) (end 135.89 89.535) (width 0.75) (layer "B.Cu") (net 4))
 (segment (start 128.27 104.2295) (end 128.27 116.84) (width 0.75) (layer "B.Cu") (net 4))
 (segment (start 144.145 89.535) (end 147.32 86.36) (width 0.75) (layer "B.Cu") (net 4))
 (segment (start 130.81 94.615) (end 130.81 97.79) (width 0.75) (layer "B.Cu") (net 4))
 (segment (start 135.89 89.535) (end 130.81 94.615) (width 0.75) (layer "B.Cu") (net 4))
 (segment (start 130.81 101.6895) (end 128.27 104.2295) (width 0.75) (layer "B.Cu") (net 4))
 (segment (start 149.225 94.52) (end 150.450497 94.52) (width 0.25) (layer "F.Cu") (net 1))
 (segment (start 150.450497 94.52) (end 150.585 94.385497) (width 0.25) (layer "F.Cu") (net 1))
 (segment (start 149.86 88.265) (end 148.59 89.535) (width 0.75) (layer "F.Cu") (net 1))
 (segment (start 147.32 81.915) (end 148.59 83.185) (width 0.25) (layer "F.Cu") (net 1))
 (segment (start 148.275 93.57) (end 149.225 94.52) (width 0.25) (layer "F.Cu") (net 1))
 (segment (start 154.94 83.185) (end 149.86 88.265) (width 0.75) (layer "F.Cu") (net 1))
 (segment (start 148.59 89.535) (end 146.685 89.535) (width 0.75) (layer "F.Cu") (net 1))
 (segment (start 150.495 88.9) (end 149.86 88.265) (width 0.25) (layer "F.Cu") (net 1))
 (segment (start 150.495 90.805) (end 150.495 88.9) (width 0.25) (layer "F.Cu") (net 1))
 (segment (start 148.59 83.185) (end 154.94 83.185) (width 0.25) (layer "F.Cu") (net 1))
 (via (at 150.585 94.385497) (size 0.8) (drill 0.4) (layers "F.Cu" "B.Cu") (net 1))
 (segment (start 154.305 83.185) (end 154.94 83.185) (width 0.75) (layer "B.Cu") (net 1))
 (segment (start 152.505 94.72) (end 152.845 94.72) (width 0.25) (layer "B.Cu") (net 1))
 (segment (start 151.765 85.725) (end 154.305 83.185) (width 0.75) (layer "B.Cu") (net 1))
 (segment (start 150.949503 94.75) (end 151.855 94.75) (width 0.25) (layer "B.Cu") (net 1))
 (segment (start 150.585 94.385497) (end 150.949503 94.75) (width 0.25) (layer "B.Cu") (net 1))
 (segment (start 153.035 94.595489) (end 153.035 92.71) (width 0.75) (layer "B.Cu") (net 1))
 (segment (start 151.765 91.44) (end 151.765 85.725) (width 0.75) (layer "B.Cu") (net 1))
 (segment (start 152.4 94.615) (end 152.505 94.72) (width 0.25) (layer "B.Cu") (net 1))
 (segment (start 151.885 94.72) (end 152.845 94.72) (width 0.25) (layer "B.Cu") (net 1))
 (segment (start 151.855 94.75) (end 151.885 94.72) (width 0.25) (layer "B.Cu") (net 1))
 (segment (start 153.035 92.71) (end 151.765 91.44) (width 0.75) (layer "B.Cu") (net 1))
 (segment (start 149.225 96.02) (end 150.220497 96.02) (width 0.2) (layer "F.Cu") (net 46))
 (segment (start 150.220497 96.02) (end 150.585 96.384503) (width 0.2) (layer "F.Cu") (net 46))
 (via (at 150.585 96.384503) (size 0.8) (drill 0.4) (layers "F.Cu" "B.Cu") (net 46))
 (segment (start 150.949503 96.02) (end 152.845 96.02) (width 0.2) (layer "B.Cu") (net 46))
 (segment (start 150.585 96.384503) (end 150.949503 96.02) (width 0.2) (layer "B.Cu") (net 46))
 (segment (start 149.225 95.52) (end 150.45 95.52) (width 0.2) (layer "F.Cu") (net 47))
 (segment (start 150.45 95.52) (end 150.585 95.385) (width 0.2) (layer "F.Cu") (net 47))
 (via (at 150.585 95.385) (size 0.8) (drill 0.4) (layers "F.Cu" "B.Cu") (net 47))
 (segment (start 150.585 95.385) (end 150.6 95.37) (width 0.2) (layer "B.Cu") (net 47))
 (segment (start 150.6 95.37) (end 152.845 95.37) (width 0.2) (layer "B.Cu") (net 47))
 (segment (start 111.6076 104.8512) (end 109.8804 103.124) (width 0.25) (layer "F.Cu") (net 5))
 (segment (start 111.623 104.8358) (end 111.6076 104.8512) (width 0.25) (layer "F.Cu") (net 5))
 (segment (start 109.8804 103.124) (end 109.8804 100.5068) (width 0.25) (layer "F.Cu") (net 5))
 (segment (start 111.6664 104.8358) (end 111.623 104.8358) (width 0.25) (layer "F.Cu") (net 5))
 (segment (start 132.309022 102.87) (end 133.774022 104.335) (width 0.25) (layer "F.Cu") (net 7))
 (segment (start 112.1664 103.5458) (end 112.3542 103.5458) (width 0.25) (layer "F.Cu") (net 7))
 (segment (start 124.46 102.87) (end 132.309022 102.87) (width 0.25) (layer "F.Cu") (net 7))
 (segment (start 112.3542 103.5458) (end 113.03 102.87) (width 0.25) (layer "F.Cu") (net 7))
 (segment (start 133.774022 104.335) (end 135.46 104.335) (width 0.25) (layer "F.Cu") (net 7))
 (via (at 124.46 102.87) (size 0.8) (drill 0.4) (layers "F.Cu" "B.Cu") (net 7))
 (via (at 113.03 102.87) (size 0.8) (drill 0.4) (layers "F.Cu" "B.Cu") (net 7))
 (segment (start 113.03 102.87) (end 124.46 102.87) (width 0.25) (layer "B.Cu") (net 7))
 (segment (start 114.935 101.1926) (end 114.1476 100.4052) (width 0.25) (layer "F.Cu") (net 6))
 (segment (start 148.275 98.47) (end 148.275 100.645) (width 0.25) (layer "F.Cu") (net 6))
 (segment (start 148.275 100.645) (end 147.955 100.965) (width 0.25) (layer "F.Cu") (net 6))
 (segment (start 114.1476 103.3546) (end 114.1476 100.4052) (width 0.25) (layer "F.Cu") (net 6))
 (segment (start 112.6664 104.8358) (end 114.1476 103.3546) (width 0.25) (layer "F.Cu") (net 6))
 (segment (start 114.935 101.6) (end 114.935 101.1926) (width 0.25) (layer "F.Cu") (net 6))
 (via (at 114.935 101.6) (size 0.8) (drill 0.4) (layers "F.Cu" "B.Cu") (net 6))
 (via (at 147.955 100.965) (size 0.8) (drill 0.4) (layers "F.Cu" "B.Cu") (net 6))
 (segment (start 147.955 100.965) (end 115.57 100.965) (width 0.25) (layer "B.Cu") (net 6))
 (segment (start 115.57 100.965) (end 114.935 101.6) (width 0.25) (layer "B.Cu") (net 6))
 (segment (start 112.1664 96.774) (end 112.1664 96.0976) (width 0.25) (layer "F.Cu") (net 11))
 (segment (start 114.1476 98.7552) (end 112.1664 96.774) (width 0.25) (layer "F.Cu") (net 11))
 (segment (start 146.275 99.47) (end 146.05 99.695) (width 0.25) (layer "F.Cu") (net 8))
 (segment (start 110.498 95.5976) (end 110.8764 95.5976) (width 0.25) (layer "F.Cu") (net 8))
 (segment (start 109.8804 96.2152) (end 110.498 95.5976) (width 0.25) (layer "F.Cu") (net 8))
 (segment (start 146.275 98.47) (end 146.275 99.47) (width 0.25) (layer "F.Cu") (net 8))
 (segment (start 110.8764 97.5414) (end 110.8764 95.5976) (width 0.25) (layer "F.Cu") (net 8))
 (segment (start 111.76 98.425) (end 110.8764 97.5414) (width 0.25) (layer "F.Cu") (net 8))
 (segment (start 109.8804 98.8568) (end 109.8804 96.2152) (width 0.25) (layer "F.Cu") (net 8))
 (via (at 111.76 98.425) (size 0.8) (drill 0.4) (layers "F.Cu" "B.Cu") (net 8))
 (via (at 146.05 99.695) (size 0.8) (drill 0.4) (layers "F.Cu" "B.Cu") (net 8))
 (segment (start 113.03 99.695) (end 111.76 98.425) (width 0.25) (layer "B.Cu") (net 8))
 (segment (start 146.05 99.695) (end 113.03 99.695) (width 0.25) (layer "B.Cu") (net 8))
 (segment (start 116.205 114.68) (end 116.575 115.05) (width 0.25) (layer "F.Cu") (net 16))
 (segment (start 116.575 115.05) (end 124.3925 115.05) (width 0.25) (layer "F.Cu") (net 16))
 (segment (start 116.4336 107.0911) (end 116.4336 106.9086) (width 0.25) (layer "F.Cu") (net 16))
 (segment (start 117.21 97.985) (end 116.4336 98.7614) (width 0.25) (layer "F.Cu") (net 16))
 (segment (start 124.3925 115.05) (end 116.4336 107.0911) (width 0.25) (layer "F.Cu") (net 16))
 (segment (start 116.4336 98.7614) (end 116.4336 106.9086) (width 0.25) (layer "F.Cu") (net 16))
 (segment (start 118.46 97.985) (end 117.21 97.985) (width 0.25) (layer "F.Cu") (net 16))
 (segment (start 147.775 93.020978) (end 147.775 93.57) (width 0.25) (layer "F.Cu") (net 43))
 (segment (start 148.845 91.950978) (end 147.775 93.020978) (width 0.25) (layer "F.Cu") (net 43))
 (segment (start 148.845 90.805) (end 148.845 91.950978) (width 0.25) (layer "F.Cu") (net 43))
 (segment (start 118.46 96.715) (end 115.7306 96.715) (width 0.25) (layer "F.Cu") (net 10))
 (segment (start 115.7224 96.7232) (end 115.7224 103.378) (width 0.25) (layer "F.Cu") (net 10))
 (segment (start 115.7306 96.715) (end 115.7224 96.7232) (width 0.25) (layer "F.Cu") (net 10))
 (segment (start 115.7224 103.378) (end 112.5728 106.5276) (width 0.25) (layer "F.Cu") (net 10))
 (segment (start 112.5728 106.5276) (end 108.458 106.5276) (width 0.25) (layer "F.Cu") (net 10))
 (via (at 108.458 106.5276) (size 0.8) (drill 0.4) (layers "F.Cu" "B.Cu") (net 10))
 (segment (start 108.458 106.5276) (end 108.3056 106.68) (width 0.25) (layer "B.Cu") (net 10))
 (segment (start 108.3056 106.68) (end 101.6 106.68) (width 0.25) (layer "B.Cu") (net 10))
 (segment (start 147.275 100.375717) (end 146.781686 100.869031) (width 0.25) (layer "F.Cu") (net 39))
 (segment (start 142.42548 99.881197) (end 142.42548 96.071198) (width 0.25) (layer "F.Cu") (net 39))
 (segment (start 139.259282 92.905) (end 135.46 92.905) (width 0.25) (layer "F.Cu") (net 39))
 (segment (start 147.275 98.47) (end 147.275 100.375717) (width 0.25) (layer "F.Cu") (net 39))
 (segment (start 146.781686 100.869031) (end 143.413314 100.869031) (width 0.25) (layer "F.Cu") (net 39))
 (segment (start 142.42548 96.071198) (end 139.259282 92.905) (width 0.25) (layer "F.Cu") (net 39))
 (segment (start 143.413314 100.869031) (end 142.42548 99.881197) (width 0.25) (layer "F.Cu") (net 39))
 (segment (start 142.875 99.695) (end 143.599511 100.419511) (width 0.25) (layer "F.Cu") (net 40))
 (segment (start 138.625 91.635) (end 142.875 95.885) (width 0.25) (layer "F.Cu") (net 40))
 (segment (start 135.46 91.635) (end 138.625 91.635) (width 0.25) (layer "F.Cu") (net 40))
 (segment (start 142.875 95.885) (end 142.875 99.695) (width 0.25) (layer "F.Cu") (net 40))
 (segment (start 143.599511 100.419511) (end 146.595489 100.419511) (width 0.25) (layer "F.Cu") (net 40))
 (segment (start 146.775 100.24) (end 146.775 98.47) (width 0.25) (layer "F.Cu") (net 40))
 (segment (start 146.595489 100.419511) (end 146.775 100.24) (width 0.25) (layer "F.Cu") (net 40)))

